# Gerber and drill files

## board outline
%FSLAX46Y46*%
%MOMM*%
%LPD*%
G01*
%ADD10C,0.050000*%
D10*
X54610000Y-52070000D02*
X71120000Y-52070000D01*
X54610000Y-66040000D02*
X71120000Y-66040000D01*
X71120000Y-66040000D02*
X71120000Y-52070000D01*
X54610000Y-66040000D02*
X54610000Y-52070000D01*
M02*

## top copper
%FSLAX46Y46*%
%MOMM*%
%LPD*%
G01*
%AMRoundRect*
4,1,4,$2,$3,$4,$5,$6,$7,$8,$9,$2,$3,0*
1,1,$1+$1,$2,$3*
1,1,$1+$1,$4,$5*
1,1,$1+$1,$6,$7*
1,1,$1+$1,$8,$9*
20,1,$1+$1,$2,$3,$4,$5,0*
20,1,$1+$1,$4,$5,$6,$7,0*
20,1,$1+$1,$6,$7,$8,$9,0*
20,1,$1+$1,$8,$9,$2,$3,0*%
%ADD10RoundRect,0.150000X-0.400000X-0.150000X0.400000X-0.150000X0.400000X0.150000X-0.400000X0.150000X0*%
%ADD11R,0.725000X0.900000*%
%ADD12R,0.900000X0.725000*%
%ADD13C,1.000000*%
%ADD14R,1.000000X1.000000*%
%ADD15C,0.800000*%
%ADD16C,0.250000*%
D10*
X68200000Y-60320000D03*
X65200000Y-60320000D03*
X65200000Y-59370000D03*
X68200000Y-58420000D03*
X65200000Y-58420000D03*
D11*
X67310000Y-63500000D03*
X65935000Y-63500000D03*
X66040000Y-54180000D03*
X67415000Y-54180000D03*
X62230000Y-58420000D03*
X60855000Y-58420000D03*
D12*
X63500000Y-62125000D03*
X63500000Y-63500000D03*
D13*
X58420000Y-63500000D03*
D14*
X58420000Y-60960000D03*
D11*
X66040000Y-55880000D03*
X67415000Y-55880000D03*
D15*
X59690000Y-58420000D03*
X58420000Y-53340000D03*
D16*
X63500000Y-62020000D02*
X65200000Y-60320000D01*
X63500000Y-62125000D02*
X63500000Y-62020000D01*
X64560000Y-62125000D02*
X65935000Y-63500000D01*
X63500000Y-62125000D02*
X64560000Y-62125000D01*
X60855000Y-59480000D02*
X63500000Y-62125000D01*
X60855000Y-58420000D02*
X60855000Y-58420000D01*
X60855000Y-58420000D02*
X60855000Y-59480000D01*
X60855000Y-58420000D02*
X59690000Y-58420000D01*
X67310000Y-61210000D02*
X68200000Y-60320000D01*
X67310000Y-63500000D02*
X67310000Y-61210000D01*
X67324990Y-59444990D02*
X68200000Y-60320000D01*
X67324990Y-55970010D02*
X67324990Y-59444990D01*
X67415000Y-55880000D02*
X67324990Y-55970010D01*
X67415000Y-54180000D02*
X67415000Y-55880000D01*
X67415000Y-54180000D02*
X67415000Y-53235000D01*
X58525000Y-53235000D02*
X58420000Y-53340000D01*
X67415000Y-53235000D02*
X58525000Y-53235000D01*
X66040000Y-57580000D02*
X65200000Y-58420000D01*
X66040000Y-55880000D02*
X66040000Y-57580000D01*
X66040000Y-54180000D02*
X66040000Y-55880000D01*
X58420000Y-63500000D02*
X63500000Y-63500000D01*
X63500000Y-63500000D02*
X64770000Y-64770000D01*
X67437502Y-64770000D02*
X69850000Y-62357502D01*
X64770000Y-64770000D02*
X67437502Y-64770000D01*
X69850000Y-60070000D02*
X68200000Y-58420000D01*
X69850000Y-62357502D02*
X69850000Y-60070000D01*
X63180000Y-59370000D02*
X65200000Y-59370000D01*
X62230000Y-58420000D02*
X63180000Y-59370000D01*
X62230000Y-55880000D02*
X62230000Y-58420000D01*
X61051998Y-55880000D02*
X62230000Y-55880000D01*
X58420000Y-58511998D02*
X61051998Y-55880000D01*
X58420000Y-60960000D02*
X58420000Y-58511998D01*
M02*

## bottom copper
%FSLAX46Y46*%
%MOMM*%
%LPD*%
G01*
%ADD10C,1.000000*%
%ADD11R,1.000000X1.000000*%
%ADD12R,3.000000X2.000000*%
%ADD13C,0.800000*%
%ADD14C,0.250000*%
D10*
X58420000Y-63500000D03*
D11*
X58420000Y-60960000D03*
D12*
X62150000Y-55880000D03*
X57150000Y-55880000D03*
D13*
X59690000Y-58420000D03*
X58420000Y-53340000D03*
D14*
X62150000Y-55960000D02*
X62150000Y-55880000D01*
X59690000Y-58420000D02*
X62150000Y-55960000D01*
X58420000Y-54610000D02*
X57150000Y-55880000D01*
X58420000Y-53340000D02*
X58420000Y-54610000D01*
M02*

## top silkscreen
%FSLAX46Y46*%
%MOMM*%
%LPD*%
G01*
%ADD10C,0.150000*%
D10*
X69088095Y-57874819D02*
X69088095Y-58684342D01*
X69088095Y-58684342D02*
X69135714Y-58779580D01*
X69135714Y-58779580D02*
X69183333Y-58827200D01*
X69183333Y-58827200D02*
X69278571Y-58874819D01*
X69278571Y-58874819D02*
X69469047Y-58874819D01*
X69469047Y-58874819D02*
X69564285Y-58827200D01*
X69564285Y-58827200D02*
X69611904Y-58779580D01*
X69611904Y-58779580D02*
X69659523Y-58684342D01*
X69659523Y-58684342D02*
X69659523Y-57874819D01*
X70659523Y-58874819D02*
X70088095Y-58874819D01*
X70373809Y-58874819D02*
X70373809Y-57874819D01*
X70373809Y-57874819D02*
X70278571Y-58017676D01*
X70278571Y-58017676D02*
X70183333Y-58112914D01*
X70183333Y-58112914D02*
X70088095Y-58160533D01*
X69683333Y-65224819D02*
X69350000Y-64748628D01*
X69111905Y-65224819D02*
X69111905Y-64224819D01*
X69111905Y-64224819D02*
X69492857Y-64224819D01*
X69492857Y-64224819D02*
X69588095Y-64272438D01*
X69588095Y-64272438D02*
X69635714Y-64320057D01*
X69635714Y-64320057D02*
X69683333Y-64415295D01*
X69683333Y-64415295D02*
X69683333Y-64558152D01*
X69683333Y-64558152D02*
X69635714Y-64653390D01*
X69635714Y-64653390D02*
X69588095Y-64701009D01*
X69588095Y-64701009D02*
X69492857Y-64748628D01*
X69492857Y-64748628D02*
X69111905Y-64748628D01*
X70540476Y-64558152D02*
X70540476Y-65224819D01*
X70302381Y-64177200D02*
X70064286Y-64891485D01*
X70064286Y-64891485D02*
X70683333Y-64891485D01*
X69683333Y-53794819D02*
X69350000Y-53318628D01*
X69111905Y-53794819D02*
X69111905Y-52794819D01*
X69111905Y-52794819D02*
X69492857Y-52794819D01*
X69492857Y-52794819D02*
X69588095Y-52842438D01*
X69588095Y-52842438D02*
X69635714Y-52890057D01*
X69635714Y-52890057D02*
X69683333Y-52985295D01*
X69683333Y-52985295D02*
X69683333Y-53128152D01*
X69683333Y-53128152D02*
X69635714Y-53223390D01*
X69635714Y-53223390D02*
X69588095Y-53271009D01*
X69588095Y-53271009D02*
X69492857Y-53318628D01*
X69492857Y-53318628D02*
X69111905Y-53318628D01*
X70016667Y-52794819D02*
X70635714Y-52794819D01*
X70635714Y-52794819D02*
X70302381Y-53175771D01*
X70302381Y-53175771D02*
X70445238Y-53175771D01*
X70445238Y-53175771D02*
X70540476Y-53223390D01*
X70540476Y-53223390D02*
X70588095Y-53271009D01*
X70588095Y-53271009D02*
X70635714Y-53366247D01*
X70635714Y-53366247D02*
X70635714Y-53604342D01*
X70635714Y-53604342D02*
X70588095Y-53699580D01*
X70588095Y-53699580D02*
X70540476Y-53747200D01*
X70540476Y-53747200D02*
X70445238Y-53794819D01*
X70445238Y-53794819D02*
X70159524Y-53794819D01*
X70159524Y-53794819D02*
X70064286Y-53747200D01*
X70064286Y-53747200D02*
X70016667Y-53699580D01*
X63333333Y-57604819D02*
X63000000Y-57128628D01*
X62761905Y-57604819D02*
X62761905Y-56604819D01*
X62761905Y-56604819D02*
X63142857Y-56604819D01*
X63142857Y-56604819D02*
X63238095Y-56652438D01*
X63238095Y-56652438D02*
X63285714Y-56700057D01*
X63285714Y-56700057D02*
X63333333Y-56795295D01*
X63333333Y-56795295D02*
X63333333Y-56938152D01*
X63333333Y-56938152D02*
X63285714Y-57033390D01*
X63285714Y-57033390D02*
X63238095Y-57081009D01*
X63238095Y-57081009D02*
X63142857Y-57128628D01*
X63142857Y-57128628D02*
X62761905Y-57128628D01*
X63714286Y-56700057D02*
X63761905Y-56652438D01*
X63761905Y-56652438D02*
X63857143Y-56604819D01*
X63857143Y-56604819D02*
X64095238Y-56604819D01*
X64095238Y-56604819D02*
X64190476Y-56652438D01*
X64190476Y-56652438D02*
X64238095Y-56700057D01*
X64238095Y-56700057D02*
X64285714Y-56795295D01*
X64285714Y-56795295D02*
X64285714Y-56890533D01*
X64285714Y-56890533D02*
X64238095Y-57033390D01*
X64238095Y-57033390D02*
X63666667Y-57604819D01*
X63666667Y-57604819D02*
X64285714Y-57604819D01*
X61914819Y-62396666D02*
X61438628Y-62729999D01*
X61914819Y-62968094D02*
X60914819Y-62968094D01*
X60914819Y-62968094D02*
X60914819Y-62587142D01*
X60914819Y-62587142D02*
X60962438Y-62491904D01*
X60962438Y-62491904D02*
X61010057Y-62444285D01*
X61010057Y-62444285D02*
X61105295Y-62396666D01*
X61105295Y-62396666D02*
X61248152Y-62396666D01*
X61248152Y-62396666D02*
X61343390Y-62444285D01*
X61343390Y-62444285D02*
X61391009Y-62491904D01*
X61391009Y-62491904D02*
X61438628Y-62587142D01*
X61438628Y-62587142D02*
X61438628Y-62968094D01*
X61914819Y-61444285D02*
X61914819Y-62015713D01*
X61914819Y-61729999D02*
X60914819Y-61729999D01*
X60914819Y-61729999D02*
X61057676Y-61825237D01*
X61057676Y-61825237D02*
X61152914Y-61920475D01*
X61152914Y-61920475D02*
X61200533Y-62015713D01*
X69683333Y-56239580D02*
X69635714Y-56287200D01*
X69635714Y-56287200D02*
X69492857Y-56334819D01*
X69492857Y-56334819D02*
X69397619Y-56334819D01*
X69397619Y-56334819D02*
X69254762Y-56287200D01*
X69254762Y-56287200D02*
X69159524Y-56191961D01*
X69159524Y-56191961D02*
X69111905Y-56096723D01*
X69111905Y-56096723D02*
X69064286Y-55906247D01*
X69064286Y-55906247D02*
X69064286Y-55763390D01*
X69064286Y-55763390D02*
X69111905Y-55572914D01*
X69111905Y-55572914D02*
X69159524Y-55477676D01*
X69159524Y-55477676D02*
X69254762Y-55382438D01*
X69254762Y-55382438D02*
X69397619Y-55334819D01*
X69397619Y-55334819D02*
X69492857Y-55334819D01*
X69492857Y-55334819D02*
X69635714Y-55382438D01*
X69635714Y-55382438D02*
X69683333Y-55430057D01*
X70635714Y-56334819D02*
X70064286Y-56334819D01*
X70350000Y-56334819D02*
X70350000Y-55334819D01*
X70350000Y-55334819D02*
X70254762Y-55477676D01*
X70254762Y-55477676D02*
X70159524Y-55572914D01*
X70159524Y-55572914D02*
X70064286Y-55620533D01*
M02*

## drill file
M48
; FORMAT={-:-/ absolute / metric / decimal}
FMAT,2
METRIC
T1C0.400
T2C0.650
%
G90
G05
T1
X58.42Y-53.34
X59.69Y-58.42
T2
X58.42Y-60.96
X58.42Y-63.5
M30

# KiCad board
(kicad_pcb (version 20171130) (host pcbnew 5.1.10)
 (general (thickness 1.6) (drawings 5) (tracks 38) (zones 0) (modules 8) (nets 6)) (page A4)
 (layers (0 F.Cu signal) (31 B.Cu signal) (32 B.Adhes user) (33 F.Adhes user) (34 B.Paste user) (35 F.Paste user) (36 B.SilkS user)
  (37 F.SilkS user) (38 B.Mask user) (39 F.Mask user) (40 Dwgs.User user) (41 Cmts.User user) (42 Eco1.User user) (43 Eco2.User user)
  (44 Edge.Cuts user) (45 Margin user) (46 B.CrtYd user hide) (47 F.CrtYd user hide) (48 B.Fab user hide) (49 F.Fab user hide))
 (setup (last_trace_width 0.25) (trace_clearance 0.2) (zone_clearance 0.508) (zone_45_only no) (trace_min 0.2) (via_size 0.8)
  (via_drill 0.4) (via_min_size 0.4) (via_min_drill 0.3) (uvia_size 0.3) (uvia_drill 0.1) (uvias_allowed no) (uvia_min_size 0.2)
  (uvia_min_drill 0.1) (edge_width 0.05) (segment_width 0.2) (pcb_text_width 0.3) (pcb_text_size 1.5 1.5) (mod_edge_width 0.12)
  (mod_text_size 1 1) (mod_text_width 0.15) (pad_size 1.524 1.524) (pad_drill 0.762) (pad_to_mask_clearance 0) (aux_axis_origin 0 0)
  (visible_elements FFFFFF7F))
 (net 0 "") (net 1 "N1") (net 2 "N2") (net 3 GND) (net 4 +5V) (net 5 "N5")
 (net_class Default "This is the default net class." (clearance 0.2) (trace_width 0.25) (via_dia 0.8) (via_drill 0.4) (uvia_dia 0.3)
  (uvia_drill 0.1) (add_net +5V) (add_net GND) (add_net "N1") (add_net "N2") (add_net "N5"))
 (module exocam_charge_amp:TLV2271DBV (layer F.Cu) (at 66.47 55.88)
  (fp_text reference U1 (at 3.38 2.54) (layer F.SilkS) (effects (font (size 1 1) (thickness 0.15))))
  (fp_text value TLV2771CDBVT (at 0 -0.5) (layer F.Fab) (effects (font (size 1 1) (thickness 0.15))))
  (pad 4 smd roundrect (at 1.73 4.44) (size 1.1 0.6) (layers F.Cu F.Paste F.Mask) (roundrect_rratio 0.25) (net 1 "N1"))
  (pad 3 smd roundrect (at -1.27 4.44) (size 1.1 0.6) (layers F.Cu F.Paste F.Mask) (roundrect_rratio 0.25) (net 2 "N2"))
  (pad 2 smd roundrect (at -1.27 3.49) (size 1.1 0.6) (layers F.Cu F.Paste F.Mask) (roundrect_rratio 0.25) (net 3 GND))
  (pad 5 smd roundrect (at 1.73 2.54) (size 1.1 0.6) (layers F.Cu F.Paste F.Mask) (roundrect_rratio 0.25) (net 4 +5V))
  (pad 1 smd roundrect (at -1.27 2.54) (size 1.1 0.6) (layers F.Cu F.Paste F.Mask) (roundrect_rratio 0.25) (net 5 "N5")))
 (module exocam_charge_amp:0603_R (layer F.Cu) (at 67.205 60.96)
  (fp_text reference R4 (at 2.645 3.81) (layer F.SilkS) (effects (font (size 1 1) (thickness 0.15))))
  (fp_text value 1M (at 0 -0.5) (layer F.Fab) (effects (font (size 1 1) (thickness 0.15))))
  (pad 2 smd rect (at 0.105 2.54) (size 0.725 0.9) (layers F.Cu F.Paste F.Mask) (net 1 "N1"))
  (pad 1 smd rect (at -1.27 2.54) (size 0.725 0.9) (layers F.Cu F.Paste F.Mask) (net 2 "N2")))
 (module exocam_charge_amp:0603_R (layer F.Cu) (at 66.145 56.72 180)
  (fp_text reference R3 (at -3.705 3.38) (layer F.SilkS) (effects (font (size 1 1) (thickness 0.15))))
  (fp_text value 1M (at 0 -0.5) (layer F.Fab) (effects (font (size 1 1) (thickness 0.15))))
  (pad 2 smd rect (at 0.105 2.54 180) (size 0.725 0.9) (layers F.Cu F.Paste F.Mask) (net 5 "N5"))
  (pad 1 smd rect (at -1.27 2.54 180) (size 0.725 0.9) (layers F.Cu F.Paste F.Mask) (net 1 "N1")))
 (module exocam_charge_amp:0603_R (layer F.Cu) (at 62.125 55.88)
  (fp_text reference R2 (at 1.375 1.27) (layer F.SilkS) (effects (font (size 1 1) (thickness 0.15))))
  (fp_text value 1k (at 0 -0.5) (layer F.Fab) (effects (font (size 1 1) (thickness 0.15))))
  (pad 2 smd rect (at 0.105 2.54) (size 0.725 0.9) (layers F.Cu F.Paste F.Mask) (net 3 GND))
  (pad 1 smd rect (at -1.27 2.54) (size 0.725 0.9) (layers F.Cu F.Paste F.Mask) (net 2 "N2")))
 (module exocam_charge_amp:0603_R (layer F.Cu) (at 60.96 62.23 90)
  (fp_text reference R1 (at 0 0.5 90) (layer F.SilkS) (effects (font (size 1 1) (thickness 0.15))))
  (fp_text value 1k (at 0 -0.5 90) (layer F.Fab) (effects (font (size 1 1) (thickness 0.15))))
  (pad 2 smd rect (at 0.105 2.54 90) (size 0.725 0.9) (layers F.Cu F.Paste F.Mask) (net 2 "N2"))
  (pad 1 smd rect (at -1.27 2.54 90) (size 0.725 0.9) (layers F.Cu F.Paste F.Mask) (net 4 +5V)))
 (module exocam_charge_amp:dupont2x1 (layer B.Cu) (at 55.88 63.5 270)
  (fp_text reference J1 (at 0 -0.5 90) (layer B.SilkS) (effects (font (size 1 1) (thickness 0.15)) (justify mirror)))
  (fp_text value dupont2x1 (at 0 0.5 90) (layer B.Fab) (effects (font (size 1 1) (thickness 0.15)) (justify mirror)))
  (pad 2 thru_hole circle (at 0 -2.54 270) (size 1 1) (drill 0.65) (layers *.Cu *.Mask) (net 4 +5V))
  (pad 1 thru_hole rect (at -2.54 -2.54 270) (size 1 1) (drill 0.65) (layers *.Cu *.Mask) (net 3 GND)))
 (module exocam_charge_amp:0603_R (layer F.Cu) (at 66.145 58.42 180)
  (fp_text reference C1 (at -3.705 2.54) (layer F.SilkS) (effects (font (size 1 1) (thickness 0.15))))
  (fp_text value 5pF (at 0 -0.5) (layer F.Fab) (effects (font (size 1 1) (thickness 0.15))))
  (pad 2 smd rect (at 0.105 2.54 180) (size 0.725 0.9) (layers F.Cu F.Paste F.Mask) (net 5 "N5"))
  (pad 1 smd rect (at -1.27 2.54 180) (size 0.725 0.9) (layers F.Cu F.Paste F.Mask) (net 1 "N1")))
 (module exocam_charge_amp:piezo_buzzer (layer B.Cu) (at 59.69 58.42)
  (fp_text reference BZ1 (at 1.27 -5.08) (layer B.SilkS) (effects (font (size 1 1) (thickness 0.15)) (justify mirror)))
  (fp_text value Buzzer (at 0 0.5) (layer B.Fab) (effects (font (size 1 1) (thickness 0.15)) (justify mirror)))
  (pad 2 smd rect (at 2.46 -2.54) (size 3 2) (layers B.Cu B.Paste B.Mask) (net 2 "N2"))
  (pad 1 smd rect (at -2.54 -2.54) (size 3 2) (layers B.Cu B.Paste B.Mask) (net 1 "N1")))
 (gr_line (start 54.61 52.07) (end 71.12 52.07) (layer Edge.Cuts) (width 0.05))
 (gr_line (start 54.61 66.04) (end 71.12 66.04) (layer Edge.Cuts) (width 0.05))
 (gr_line (start 71.12 66.04) (end 71.12 52.07) (layer Edge.Cuts) (width 0.05))
 (gr_line (start 54.61 66.04) (end 54.61 52.07) (layer Edge.Cuts) (width 0.05))
 (segment (start 63.5 62.02) (end 65.2 60.32) (width 0.25) (layer F.Cu) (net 2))
 (segment (start 63.5 62.125) (end 63.5 62.02) (width 0.25) (layer F.Cu) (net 2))
 (segment (start 64.56 62.125) (end 65.935 63.5) (width 0.25) (layer F.Cu) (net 2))
 (segment (start 63.5 62.125) (end 64.56 62.125) (width 0.25) (layer F.Cu) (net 2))
 (segment (start 60.855 59.48) (end 63.5 62.125) (width 0.25) (layer F.Cu) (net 2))
 (segment (start 60.855 58.42) (end 60.855 58.42) (width 0.25) (layer F.Cu) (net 2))
 (segment (start 60.855 58.42) (end 60.855 59.48) (width 0.25) (layer F.Cu) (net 2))
 (via (at 59.69 58.42) (size 0.8) (drill 0.4) (layers F.Cu B.Cu) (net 2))
 (segment (start 60.855 58.42) (end 59.69 58.42) (width 0.25) (layer F.Cu) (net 2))
 (segment (start 62.15 55.96) (end 62.15 55.88) (width 0.25) (layer B.Cu) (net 2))
 (segment (start 59.69 58.42) (end 62.15 55.96) (width 0.25) (layer B.Cu) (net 2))
 (via (at 58.42 53.34) (size 0.8) (drill 0.4) (layers F.Cu B.Cu) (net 1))
 (segment (start 67.31 61.21) (end 68.2 60.32) (width 0.25) (layer F.Cu) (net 1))
 (segment (start 67.31 63.5) (end 67.31 61.21) (width 0.25) (layer F.Cu) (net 1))
 (segment (start 67.32499 59.44499) (end 68.2 60.32) (width 0.25) (layer F.Cu) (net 1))
 (segment (start 67.32499 55.97001) (end 67.32499 59.44499) (width 0.25) (layer F.Cu) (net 1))
 (segment (start 67.415 55.88) (end 67.32499 55.97001) (width 0.25) (layer F.Cu) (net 1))
 (segment (start 67.415 54.18) (end 67.415 55.88) (width 0.25) (layer F.Cu) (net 1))
 (segment (start 67.415 54.18) (end 67.415 53.235) (width 0.25) (layer F.Cu) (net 1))
 (segment (start 58.525 53.235) (end 58.42 53.34) (width 0.25) (layer F.Cu) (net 1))
 (segment (start 67.415 53.235) (end 58.525 53.235) (width 0.25) (layer F.Cu) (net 1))
 (segment (start 58.42 54.61) (end 57.15 55.88) (width 0.25) (layer B.Cu) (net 1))
 (segment (start 58.42 53.34) (end 58.42 54.61) (width 0.25) (layer B.Cu) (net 1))
 (segment (start 66.04 57.58) (end 65.2 58.42) (width 0.25) (layer F.Cu) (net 5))
 (segment (start 66.04 55.88) (end 66.04 57.58) (width 0.25) (layer F.Cu) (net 5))
 (segment (start 66.04 54.18) (end 66.04 55.88) (width 0.25) (layer F.Cu) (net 5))
 (segment (start 58.42 63.5) (end 63.5 63.5) (width 0.25) (layer F.Cu) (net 4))
 (segment (start 63.5 63.5) (end 64.77 64.77) (width 0.25) (layer F.Cu) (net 4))
 (segment (start 67.437502 64.77) (end 69.85 62.357502) (width 0.25) (layer F.Cu) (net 4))
 (segment (start 64.77 64.77) (end 67.437502 64.77) (width 0.25) (layer F.Cu) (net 4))
 (segment (start 69.85 60.07) (end 68.2 58.42) (width 0.25) (layer F.Cu) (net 4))
 (segment (start 69.85 62.357502) (end 69.85 60.07) (width 0.25) (layer F.Cu) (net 4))
 (segment (start 63.18 59.37) (end 65.2 59.37) (width 0.25) (layer F.Cu) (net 3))
 (segment (start 62.23 58.42) (end 63.18 59.37) (width 0.25) (layer F.Cu) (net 3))
 (segment (start 62.23 55.88) (end 62.23 58.42) (width 0.25) (layer F.Cu) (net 3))
 (segment (start 61.051998 55.88) (end 62.23 55.88) (width 0.25) (layer F.Cu) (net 3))
 (segment (start 58.42 58.511998) (end 61.051998 55.88) (width 0.25) (layer F.Cu) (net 3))
 (segment (start 58.42 60.96) (end 58.42 58.511998) (width 0.25) (layer F.Cu) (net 3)))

